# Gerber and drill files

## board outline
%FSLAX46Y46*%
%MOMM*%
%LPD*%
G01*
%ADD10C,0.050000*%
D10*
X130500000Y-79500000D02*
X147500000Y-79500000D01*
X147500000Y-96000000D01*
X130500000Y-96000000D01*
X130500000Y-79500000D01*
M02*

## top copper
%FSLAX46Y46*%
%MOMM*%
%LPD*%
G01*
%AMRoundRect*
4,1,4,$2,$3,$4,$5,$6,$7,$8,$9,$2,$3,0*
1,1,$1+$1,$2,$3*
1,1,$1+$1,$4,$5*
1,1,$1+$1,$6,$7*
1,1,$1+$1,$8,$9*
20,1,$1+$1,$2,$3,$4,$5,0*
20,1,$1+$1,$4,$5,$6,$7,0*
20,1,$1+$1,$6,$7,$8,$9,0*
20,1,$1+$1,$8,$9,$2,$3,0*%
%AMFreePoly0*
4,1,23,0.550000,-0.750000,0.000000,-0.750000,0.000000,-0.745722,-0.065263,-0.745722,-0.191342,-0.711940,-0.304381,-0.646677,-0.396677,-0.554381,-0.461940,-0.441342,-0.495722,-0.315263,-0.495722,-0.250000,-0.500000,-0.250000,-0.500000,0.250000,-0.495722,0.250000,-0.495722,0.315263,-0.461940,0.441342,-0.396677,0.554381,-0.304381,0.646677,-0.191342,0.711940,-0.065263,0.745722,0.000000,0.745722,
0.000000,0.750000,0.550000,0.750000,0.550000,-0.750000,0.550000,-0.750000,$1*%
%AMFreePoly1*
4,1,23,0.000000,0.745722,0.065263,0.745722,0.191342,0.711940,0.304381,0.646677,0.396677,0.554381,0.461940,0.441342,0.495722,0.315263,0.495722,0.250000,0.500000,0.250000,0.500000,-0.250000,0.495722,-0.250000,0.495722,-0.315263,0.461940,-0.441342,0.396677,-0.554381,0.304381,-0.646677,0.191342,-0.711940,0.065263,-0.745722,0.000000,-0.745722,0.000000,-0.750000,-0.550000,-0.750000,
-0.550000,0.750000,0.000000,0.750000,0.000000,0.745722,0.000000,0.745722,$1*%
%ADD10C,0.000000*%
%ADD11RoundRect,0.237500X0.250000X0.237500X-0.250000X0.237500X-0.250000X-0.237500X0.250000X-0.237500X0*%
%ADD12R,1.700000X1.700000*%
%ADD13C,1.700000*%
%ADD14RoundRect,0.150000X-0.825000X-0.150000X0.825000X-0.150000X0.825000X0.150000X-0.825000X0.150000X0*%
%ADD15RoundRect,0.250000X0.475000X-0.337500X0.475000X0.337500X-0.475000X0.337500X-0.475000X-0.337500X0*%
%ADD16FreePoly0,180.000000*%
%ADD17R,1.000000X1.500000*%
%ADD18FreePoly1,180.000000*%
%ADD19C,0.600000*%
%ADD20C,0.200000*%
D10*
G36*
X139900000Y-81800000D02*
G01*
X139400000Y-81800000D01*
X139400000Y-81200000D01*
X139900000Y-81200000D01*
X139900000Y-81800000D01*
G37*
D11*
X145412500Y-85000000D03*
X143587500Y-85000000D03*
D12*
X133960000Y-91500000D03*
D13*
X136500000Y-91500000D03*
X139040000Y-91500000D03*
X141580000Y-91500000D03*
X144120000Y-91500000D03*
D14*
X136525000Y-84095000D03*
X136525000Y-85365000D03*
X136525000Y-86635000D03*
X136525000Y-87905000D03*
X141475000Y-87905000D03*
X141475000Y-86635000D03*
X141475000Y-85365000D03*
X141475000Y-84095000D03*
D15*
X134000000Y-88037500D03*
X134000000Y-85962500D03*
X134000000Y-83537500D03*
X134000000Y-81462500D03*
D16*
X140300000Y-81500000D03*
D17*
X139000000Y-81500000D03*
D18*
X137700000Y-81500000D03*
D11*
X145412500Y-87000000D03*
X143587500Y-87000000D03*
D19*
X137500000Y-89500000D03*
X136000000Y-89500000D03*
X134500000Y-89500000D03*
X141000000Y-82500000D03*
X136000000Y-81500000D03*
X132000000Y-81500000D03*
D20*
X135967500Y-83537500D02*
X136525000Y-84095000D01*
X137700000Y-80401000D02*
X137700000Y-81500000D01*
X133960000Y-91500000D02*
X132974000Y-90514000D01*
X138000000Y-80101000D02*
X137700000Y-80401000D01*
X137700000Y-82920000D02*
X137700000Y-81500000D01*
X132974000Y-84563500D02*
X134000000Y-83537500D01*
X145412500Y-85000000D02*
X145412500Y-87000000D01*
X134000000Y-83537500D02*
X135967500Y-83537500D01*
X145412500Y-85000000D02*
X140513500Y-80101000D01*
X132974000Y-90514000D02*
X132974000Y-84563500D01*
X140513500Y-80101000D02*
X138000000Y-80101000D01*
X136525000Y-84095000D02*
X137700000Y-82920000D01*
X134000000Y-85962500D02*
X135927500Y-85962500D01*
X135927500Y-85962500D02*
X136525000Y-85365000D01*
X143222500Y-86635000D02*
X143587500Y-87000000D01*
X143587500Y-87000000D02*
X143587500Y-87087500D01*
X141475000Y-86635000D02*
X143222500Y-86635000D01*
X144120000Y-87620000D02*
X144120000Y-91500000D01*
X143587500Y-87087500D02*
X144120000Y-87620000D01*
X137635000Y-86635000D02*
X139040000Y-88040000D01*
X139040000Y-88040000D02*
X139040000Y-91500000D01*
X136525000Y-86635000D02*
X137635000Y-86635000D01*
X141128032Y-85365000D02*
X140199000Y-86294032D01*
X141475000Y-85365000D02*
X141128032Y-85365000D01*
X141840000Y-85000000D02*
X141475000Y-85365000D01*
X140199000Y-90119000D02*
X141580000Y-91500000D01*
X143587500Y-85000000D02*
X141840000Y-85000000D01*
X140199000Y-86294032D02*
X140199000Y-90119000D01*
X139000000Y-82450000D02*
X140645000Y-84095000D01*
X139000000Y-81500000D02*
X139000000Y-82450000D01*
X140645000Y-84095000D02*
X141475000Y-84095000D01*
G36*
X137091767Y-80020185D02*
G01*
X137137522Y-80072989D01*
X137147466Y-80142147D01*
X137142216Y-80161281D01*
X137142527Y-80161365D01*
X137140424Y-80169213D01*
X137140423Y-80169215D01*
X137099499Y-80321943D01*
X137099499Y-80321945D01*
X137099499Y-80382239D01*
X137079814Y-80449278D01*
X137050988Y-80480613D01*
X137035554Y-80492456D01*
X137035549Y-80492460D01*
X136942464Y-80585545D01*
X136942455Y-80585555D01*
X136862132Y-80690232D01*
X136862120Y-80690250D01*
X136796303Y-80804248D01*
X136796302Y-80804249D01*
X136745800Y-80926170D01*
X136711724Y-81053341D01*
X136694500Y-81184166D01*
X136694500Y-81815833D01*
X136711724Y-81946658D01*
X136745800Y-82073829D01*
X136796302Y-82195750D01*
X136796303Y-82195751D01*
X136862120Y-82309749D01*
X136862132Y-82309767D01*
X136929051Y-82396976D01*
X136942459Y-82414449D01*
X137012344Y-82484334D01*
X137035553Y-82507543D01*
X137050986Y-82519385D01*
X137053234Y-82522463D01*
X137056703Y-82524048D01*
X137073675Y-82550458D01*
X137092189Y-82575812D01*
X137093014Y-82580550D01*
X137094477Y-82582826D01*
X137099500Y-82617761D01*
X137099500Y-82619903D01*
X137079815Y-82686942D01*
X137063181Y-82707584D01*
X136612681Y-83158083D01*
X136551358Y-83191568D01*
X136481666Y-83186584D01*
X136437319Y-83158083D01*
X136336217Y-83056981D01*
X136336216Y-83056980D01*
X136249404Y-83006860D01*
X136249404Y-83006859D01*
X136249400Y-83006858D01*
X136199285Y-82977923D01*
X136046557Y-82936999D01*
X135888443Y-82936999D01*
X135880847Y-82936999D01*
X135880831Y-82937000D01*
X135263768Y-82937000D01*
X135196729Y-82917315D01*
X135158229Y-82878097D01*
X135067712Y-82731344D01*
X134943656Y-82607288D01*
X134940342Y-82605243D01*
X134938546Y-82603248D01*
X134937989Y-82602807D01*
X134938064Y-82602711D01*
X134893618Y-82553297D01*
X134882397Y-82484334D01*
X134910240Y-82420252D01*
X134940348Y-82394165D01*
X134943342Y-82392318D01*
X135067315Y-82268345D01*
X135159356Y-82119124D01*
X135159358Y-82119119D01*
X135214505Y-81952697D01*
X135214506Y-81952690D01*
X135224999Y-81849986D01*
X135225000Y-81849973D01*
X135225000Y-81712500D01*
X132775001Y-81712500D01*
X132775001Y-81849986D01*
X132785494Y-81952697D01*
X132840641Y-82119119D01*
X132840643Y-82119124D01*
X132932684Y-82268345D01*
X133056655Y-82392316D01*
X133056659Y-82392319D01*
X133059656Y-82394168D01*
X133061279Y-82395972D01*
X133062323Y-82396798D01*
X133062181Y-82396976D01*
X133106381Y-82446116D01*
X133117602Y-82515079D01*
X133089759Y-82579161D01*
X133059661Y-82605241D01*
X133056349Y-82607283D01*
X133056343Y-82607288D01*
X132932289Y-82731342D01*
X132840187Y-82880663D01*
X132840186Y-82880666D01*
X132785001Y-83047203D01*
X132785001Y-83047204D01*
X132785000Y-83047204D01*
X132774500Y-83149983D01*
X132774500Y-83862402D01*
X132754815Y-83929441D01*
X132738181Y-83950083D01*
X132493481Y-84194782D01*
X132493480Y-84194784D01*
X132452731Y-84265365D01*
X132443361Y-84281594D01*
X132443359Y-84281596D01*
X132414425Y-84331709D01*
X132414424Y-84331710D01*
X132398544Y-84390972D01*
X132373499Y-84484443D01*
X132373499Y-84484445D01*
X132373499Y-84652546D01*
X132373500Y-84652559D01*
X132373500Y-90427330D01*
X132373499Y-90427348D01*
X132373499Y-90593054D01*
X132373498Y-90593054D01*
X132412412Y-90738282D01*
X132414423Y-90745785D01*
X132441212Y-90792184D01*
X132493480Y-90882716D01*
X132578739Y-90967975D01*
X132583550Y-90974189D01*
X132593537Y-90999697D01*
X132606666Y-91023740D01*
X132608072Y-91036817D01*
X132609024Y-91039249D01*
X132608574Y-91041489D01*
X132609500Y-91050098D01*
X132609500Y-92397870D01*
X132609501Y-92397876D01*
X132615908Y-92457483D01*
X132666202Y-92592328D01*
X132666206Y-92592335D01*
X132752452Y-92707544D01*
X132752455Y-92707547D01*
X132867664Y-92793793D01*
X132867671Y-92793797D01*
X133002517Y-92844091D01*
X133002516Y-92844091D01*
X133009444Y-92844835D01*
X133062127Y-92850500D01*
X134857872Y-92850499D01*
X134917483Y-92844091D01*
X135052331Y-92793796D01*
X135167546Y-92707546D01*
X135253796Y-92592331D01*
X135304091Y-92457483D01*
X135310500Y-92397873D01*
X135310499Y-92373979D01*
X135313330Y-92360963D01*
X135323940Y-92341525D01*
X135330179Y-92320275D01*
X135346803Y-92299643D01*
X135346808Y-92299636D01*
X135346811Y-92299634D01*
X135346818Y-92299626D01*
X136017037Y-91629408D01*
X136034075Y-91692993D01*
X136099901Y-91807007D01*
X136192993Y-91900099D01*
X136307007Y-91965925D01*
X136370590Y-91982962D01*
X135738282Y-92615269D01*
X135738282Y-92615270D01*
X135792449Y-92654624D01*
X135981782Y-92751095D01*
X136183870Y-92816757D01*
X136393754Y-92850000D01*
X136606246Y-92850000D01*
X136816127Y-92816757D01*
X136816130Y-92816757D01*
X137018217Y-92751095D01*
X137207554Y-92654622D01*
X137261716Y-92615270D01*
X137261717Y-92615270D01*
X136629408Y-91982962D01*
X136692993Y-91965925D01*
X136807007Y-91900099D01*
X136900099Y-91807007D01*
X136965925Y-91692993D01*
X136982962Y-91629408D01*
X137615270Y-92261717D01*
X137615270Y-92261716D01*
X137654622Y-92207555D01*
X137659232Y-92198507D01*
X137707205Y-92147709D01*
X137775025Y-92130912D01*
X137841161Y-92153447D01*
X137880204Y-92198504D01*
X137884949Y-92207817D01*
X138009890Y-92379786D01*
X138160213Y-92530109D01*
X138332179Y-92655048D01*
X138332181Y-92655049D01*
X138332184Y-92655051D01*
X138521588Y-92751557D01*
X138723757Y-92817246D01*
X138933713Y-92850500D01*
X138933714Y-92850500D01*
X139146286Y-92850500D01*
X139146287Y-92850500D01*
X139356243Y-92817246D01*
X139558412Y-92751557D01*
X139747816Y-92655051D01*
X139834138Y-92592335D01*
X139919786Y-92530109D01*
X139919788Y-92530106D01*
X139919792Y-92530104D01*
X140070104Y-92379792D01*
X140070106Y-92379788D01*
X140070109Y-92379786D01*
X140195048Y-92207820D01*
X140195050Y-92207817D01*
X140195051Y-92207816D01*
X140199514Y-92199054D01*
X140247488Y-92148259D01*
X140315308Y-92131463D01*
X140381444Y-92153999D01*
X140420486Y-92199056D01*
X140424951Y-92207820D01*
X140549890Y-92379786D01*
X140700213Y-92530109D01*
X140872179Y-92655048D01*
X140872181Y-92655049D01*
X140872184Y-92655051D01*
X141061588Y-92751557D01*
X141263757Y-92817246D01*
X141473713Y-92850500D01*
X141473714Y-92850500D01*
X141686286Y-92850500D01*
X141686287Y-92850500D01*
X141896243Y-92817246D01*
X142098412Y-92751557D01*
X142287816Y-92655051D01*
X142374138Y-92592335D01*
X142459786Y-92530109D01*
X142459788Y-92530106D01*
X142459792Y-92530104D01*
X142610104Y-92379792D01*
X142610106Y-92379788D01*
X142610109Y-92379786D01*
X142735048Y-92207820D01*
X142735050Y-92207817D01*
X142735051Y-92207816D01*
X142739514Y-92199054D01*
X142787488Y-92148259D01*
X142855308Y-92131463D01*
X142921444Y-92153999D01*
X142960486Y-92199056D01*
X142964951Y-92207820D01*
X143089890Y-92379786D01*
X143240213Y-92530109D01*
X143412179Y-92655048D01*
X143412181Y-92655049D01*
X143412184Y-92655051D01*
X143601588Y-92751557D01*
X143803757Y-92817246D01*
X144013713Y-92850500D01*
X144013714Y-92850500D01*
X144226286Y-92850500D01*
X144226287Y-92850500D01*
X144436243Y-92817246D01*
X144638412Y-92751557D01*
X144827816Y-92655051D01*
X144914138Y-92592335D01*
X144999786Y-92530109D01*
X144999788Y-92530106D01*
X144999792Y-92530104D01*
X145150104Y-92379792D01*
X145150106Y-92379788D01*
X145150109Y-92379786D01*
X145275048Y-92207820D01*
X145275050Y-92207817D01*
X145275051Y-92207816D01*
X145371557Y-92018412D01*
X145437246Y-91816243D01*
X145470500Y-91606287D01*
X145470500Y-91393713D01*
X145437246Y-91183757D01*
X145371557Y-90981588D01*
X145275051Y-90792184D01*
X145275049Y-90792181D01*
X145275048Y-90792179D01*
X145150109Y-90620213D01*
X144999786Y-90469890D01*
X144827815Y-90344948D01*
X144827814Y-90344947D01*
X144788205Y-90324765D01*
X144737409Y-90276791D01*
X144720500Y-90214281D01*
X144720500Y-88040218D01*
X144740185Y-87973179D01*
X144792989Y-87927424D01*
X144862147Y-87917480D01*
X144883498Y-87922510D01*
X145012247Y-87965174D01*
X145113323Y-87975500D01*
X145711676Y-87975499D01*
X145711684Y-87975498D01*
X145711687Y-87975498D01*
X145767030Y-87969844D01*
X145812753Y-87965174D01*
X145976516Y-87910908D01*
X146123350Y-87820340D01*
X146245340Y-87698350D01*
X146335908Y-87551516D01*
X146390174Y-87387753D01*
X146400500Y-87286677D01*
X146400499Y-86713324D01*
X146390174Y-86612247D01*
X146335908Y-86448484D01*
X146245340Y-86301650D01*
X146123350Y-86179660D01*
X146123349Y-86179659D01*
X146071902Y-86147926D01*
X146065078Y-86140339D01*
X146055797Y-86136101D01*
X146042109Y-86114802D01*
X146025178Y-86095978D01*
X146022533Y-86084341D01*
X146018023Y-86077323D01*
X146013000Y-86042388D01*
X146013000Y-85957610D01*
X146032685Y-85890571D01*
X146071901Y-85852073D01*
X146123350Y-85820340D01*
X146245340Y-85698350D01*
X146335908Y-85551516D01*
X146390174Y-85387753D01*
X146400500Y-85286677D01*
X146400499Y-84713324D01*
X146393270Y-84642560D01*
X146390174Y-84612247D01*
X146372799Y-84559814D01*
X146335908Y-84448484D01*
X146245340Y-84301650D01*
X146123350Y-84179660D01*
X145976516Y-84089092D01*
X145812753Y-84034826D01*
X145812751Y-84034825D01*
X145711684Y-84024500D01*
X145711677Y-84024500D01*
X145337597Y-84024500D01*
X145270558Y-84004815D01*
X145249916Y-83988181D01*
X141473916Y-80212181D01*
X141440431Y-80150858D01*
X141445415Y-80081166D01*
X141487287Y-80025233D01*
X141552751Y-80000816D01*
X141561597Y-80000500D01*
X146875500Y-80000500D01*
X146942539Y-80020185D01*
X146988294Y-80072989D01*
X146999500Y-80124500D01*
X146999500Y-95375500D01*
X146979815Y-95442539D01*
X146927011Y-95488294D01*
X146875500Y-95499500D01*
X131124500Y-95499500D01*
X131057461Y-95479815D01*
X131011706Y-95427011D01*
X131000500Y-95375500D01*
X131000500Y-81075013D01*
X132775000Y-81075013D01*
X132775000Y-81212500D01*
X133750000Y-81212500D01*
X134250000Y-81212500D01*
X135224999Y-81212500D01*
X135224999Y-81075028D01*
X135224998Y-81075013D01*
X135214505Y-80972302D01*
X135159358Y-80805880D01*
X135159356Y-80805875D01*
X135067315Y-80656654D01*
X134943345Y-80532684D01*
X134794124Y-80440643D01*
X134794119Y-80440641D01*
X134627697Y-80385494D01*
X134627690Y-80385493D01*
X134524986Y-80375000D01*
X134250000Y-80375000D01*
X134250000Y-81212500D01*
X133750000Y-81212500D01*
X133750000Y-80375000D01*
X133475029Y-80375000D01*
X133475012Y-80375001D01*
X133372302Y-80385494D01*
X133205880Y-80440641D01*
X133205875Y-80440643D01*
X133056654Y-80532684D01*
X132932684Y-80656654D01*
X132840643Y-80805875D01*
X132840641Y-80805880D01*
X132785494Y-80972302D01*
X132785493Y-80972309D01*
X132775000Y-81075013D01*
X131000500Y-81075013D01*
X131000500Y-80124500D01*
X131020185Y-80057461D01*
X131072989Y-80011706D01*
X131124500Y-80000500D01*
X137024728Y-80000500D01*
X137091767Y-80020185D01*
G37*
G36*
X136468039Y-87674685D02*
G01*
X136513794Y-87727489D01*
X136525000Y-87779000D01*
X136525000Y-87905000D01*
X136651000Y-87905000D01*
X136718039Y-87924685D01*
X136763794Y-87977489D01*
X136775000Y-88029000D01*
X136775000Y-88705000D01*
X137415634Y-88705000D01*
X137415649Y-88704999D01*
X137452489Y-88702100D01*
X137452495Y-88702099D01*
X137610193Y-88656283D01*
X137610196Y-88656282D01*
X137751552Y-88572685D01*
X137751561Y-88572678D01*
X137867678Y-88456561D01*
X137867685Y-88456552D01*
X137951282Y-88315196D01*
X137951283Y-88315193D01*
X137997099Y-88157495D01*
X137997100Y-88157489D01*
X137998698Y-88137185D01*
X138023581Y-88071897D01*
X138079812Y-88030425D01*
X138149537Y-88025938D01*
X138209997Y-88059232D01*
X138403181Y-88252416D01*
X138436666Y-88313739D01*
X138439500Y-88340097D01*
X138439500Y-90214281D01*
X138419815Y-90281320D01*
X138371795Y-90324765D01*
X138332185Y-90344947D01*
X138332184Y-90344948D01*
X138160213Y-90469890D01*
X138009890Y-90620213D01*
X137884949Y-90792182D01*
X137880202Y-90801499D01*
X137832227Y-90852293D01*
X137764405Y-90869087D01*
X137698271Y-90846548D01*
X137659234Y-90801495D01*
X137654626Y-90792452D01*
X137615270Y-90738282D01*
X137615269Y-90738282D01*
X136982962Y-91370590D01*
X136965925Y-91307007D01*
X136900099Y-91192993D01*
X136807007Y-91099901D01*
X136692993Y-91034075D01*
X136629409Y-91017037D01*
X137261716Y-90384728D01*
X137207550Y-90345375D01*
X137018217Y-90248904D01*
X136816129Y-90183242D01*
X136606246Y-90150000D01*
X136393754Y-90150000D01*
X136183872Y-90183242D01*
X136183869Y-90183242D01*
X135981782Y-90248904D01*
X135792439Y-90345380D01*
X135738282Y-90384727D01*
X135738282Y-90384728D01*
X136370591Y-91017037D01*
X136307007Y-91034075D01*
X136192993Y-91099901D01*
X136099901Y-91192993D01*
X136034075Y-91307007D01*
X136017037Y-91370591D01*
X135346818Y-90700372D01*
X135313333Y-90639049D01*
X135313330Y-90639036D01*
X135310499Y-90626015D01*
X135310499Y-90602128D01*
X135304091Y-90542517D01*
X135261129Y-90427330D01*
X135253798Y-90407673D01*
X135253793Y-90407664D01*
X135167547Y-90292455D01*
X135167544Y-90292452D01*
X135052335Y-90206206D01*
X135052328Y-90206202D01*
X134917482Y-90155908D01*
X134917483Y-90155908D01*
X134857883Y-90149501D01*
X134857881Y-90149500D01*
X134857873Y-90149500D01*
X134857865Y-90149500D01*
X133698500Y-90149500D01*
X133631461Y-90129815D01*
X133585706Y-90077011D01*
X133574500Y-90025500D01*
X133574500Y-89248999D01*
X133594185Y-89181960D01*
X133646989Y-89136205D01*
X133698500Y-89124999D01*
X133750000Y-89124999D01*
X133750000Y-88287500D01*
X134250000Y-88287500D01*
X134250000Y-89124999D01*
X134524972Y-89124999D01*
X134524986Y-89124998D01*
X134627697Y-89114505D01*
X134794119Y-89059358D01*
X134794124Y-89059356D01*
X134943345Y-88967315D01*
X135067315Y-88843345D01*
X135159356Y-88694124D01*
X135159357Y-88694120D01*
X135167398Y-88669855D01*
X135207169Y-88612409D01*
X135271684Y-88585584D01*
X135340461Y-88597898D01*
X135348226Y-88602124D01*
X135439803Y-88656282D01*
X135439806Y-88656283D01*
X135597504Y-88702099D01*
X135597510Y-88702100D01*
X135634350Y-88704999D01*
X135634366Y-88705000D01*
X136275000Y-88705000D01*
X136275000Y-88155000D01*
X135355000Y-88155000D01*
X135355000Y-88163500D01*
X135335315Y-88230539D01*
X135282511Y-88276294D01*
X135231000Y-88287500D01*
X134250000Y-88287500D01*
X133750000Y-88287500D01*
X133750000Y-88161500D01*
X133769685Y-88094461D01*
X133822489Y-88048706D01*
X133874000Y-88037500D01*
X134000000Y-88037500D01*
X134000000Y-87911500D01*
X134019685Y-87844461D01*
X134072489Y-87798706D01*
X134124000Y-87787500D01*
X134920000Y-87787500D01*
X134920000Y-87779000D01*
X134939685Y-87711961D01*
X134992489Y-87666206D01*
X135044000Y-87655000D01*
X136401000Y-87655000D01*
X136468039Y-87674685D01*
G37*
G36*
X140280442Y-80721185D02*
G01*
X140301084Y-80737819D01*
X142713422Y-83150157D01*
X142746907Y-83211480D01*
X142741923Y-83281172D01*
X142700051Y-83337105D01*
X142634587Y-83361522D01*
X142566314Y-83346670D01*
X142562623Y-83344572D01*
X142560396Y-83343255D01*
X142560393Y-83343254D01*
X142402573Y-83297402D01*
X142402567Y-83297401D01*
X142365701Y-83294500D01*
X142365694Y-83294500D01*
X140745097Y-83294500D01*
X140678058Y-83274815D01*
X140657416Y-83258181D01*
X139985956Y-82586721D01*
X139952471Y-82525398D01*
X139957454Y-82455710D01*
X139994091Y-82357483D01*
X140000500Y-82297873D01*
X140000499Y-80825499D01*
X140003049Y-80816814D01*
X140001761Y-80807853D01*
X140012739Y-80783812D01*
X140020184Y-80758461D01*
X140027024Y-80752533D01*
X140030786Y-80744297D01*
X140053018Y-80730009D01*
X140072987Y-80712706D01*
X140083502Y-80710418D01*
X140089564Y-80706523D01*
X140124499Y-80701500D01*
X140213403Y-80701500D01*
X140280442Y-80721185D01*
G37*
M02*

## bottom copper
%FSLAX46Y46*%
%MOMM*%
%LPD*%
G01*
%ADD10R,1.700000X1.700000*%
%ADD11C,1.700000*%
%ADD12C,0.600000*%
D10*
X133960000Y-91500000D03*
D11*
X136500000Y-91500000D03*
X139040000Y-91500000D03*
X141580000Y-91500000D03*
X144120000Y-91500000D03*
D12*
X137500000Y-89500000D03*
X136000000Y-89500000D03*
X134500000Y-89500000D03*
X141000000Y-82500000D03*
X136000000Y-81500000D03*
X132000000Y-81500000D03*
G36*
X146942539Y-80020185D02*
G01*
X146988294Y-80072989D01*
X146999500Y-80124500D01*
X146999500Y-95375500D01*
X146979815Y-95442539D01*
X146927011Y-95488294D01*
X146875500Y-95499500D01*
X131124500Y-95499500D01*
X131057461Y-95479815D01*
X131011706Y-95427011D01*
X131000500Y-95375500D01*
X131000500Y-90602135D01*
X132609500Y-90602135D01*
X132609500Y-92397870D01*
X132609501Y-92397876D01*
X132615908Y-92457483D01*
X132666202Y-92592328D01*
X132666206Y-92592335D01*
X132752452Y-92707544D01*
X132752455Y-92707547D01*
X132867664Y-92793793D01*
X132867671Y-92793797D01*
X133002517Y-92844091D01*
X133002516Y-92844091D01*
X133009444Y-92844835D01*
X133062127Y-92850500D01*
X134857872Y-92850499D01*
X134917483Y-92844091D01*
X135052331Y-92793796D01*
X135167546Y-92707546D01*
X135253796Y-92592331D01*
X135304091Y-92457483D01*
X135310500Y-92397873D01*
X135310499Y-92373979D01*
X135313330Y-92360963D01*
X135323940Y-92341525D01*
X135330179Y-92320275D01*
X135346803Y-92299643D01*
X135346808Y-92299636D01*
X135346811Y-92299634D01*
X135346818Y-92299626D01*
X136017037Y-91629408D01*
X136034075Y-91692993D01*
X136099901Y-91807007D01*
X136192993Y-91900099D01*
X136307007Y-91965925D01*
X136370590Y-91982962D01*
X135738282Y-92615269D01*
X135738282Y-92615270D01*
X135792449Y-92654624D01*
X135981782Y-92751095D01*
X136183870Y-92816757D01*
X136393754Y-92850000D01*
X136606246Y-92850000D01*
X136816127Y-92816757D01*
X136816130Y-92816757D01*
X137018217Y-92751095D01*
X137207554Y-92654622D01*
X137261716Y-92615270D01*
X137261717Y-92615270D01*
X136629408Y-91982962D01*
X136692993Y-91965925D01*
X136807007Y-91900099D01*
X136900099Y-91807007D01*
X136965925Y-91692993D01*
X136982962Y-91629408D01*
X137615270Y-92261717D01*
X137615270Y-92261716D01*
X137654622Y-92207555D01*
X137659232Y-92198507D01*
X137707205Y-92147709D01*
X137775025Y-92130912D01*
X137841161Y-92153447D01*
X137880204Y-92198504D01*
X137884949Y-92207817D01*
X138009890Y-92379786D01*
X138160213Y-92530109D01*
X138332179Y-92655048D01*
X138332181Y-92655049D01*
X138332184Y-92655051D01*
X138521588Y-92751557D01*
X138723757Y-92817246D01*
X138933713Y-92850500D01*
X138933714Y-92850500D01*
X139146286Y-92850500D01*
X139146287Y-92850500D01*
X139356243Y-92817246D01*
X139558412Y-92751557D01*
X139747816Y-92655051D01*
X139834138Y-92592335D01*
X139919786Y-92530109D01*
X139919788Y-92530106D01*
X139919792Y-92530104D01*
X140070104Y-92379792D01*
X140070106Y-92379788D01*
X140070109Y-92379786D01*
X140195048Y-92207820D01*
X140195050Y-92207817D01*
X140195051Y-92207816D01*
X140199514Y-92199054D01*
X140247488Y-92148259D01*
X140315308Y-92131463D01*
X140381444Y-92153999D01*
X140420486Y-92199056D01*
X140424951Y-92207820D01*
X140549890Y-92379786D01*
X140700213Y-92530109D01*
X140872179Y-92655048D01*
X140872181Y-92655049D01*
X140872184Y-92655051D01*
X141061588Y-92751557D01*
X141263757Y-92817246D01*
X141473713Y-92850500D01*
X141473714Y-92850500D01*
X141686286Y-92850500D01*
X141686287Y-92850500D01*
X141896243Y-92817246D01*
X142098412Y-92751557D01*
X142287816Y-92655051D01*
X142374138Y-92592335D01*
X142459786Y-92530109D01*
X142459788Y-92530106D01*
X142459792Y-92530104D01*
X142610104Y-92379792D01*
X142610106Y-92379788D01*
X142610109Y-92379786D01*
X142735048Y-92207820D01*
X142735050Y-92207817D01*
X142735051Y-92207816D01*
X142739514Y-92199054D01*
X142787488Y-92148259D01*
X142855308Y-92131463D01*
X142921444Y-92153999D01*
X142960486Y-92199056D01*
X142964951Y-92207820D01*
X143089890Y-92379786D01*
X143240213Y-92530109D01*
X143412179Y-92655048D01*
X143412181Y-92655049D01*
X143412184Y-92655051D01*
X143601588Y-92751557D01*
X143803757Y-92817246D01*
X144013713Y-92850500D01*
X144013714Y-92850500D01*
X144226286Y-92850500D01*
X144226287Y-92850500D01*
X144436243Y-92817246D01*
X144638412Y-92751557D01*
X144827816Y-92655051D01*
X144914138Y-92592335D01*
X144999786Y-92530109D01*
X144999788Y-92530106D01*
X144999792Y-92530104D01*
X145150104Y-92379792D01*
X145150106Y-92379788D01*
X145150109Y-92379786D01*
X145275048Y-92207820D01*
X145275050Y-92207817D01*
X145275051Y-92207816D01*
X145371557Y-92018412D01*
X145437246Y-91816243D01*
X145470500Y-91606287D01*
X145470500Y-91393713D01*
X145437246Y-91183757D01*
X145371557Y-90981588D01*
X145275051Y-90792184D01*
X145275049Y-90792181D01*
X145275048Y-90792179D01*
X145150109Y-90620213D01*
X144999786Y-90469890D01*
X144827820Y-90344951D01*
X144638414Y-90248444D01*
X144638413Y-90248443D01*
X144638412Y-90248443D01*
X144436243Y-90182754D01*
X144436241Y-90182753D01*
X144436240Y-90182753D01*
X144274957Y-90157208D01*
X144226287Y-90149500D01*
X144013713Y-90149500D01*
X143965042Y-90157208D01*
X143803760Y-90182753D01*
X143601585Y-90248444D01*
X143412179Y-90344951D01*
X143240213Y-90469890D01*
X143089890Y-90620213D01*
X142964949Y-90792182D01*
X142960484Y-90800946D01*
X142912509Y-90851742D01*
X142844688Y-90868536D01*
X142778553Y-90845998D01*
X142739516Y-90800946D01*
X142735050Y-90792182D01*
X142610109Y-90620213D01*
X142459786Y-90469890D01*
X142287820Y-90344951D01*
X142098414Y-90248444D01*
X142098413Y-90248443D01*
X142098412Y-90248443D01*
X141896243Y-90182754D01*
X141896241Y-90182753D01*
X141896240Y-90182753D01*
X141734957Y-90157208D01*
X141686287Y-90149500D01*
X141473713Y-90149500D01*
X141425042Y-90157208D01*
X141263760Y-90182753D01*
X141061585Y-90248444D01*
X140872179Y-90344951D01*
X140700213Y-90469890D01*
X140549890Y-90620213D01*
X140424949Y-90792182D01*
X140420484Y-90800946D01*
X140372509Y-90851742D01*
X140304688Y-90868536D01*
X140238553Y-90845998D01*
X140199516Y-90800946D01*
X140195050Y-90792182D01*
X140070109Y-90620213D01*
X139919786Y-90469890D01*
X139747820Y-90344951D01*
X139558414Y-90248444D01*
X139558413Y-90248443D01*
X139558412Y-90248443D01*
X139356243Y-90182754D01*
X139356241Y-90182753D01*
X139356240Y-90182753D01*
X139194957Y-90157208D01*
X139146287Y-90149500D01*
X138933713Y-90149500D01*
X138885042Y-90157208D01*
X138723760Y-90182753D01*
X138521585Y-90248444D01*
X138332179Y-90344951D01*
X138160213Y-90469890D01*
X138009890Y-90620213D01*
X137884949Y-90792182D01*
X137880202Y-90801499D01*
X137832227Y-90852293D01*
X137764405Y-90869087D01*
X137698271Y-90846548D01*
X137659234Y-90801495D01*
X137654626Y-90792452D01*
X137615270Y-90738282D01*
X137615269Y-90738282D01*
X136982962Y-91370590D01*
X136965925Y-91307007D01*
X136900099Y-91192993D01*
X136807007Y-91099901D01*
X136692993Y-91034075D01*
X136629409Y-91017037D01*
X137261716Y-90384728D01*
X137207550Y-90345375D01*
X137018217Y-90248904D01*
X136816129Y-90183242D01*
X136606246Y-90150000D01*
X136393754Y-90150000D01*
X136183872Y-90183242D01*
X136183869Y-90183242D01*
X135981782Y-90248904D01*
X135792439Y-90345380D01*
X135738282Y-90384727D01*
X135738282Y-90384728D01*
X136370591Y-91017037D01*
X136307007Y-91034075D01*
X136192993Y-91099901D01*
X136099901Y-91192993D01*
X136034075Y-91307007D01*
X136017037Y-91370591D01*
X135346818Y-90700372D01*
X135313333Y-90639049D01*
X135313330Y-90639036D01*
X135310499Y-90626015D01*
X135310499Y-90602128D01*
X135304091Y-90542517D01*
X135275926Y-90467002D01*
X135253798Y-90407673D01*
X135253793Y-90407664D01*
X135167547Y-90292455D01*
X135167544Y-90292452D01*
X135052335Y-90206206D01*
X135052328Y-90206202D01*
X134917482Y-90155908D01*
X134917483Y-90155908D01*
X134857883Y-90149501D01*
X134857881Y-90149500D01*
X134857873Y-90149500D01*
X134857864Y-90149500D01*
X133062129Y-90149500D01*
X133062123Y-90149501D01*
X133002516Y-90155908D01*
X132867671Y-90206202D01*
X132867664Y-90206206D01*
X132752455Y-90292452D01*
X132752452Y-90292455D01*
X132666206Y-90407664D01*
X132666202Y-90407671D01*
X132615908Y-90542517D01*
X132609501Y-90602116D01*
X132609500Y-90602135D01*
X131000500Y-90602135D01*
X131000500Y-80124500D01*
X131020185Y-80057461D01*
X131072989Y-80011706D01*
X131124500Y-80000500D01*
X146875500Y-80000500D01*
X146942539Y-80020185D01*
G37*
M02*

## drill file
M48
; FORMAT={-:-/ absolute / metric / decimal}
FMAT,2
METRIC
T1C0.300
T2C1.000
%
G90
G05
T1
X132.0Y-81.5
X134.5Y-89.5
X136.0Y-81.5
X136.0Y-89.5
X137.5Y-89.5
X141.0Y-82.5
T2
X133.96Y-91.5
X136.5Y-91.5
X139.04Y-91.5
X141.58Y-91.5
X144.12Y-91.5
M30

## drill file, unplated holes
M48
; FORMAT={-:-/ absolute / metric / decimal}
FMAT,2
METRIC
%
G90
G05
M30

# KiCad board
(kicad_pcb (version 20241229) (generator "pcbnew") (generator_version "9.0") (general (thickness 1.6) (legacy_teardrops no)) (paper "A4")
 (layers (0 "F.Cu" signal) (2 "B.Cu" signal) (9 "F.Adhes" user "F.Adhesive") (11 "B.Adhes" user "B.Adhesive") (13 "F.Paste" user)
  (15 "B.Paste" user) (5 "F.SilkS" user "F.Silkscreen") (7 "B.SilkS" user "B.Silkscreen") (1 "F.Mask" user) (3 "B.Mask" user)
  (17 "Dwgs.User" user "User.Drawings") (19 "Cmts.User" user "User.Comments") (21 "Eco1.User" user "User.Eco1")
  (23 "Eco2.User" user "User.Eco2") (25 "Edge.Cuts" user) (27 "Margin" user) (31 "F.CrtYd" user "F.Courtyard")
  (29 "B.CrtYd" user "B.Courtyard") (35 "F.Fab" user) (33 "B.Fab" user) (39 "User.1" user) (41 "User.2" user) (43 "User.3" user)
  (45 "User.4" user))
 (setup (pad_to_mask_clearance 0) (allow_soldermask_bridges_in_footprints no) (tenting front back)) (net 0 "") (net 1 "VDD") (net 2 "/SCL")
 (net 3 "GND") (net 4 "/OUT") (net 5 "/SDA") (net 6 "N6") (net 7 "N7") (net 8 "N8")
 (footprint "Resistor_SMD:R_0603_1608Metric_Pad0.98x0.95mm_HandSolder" (layer "F.Cu") (at 144.5 85 180)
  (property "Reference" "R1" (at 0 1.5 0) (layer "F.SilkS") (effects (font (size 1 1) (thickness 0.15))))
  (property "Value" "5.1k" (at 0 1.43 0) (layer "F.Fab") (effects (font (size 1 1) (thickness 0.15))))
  (pad "1" smd roundrect (at -0.9125 0 180) (size 0.975 0.95) (layers "F.Cu" "F.Mask" "F.Paste") (roundrect_rratio 0.25) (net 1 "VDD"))
  (pad "2" smd roundrect (at 0.9125 0 180) (size 0.975 0.95) (layers "F.Cu" "F.Mask" "F.Paste") (roundrect_rratio 0.25) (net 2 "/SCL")))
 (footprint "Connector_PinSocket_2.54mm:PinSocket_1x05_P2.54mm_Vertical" (layer "F.Cu") (at 133.96 91.5 90)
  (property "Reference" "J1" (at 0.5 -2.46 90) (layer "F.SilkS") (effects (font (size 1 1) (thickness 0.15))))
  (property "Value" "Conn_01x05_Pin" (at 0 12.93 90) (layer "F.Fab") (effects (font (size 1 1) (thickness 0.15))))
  (pad "1" thru_hole rect (at 0 0 90) (size 1.7 1.7) (drill 1) (layers "*.Cu" "*.Mask") (remove_unused_layers no) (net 1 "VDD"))
  (pad "2" thru_hole circle (at 0 2.54 90) (size 1.7 1.7) (drill 1) (layers "*.Cu" "*.Mask") (remove_unused_layers no) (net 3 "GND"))
  (pad "3" thru_hole circle (at 0 5.08 90) (size 1.7 1.7) (drill 1) (layers "*.Cu" "*.Mask") (remove_unused_layers no) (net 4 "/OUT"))
  (pad "4" thru_hole circle (at 0 7.62 90) (size 1.7 1.7) (drill 1) (layers "*.Cu" "*.Mask") (remove_unused_layers no) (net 2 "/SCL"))
  (pad "5" thru_hole circle (at 0 10.16 90) (size 1.7 1.7) (drill 1) (layers "*.Cu" "*.Mask") (remove_unused_layers no) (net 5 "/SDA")))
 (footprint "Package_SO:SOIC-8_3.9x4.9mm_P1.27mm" (layer "F.Cu") (at 139 86)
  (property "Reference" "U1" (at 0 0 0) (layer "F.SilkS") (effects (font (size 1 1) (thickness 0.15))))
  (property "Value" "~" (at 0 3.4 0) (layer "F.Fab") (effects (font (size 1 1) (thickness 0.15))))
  (pad "1" smd roundrect (at -2.475 -1.905) (size 1.95 0.6) (layers "F.Cu" "F.Mask" "F.Paste") (roundrect_rratio 0.25) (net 1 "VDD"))
  (pad "2" smd roundrect (at -2.475 -0.635) (size 1.95 0.6) (layers "F.Cu" "F.Mask" "F.Paste") (roundrect_rratio 0.25) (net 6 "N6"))
  (pad "3" smd roundrect (at -2.475 0.635) (size 1.95 0.6) (layers "F.Cu" "F.Mask" "F.Paste") (roundrect_rratio 0.25) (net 4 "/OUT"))
  (pad "4" smd roundrect (at -2.475 1.905) (size 1.95 0.6) (layers "F.Cu" "F.Mask" "F.Paste") (roundrect_rratio 0.25) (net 3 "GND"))
  (pad "5" smd roundrect (at 2.475 1.905) (size 1.95 0.6) (layers "F.Cu" "F.Mask" "F.Paste") (roundrect_rratio 0.25) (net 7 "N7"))
  (pad "6" smd roundrect (at 2.475 0.635) (size 1.95 0.6) (layers "F.Cu" "F.Mask" "F.Paste") (roundrect_rratio 0.25) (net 5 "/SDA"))
  (pad "7" smd roundrect (at 2.475 -0.635) (size 1.95 0.6) (layers "F.Cu" "F.Mask" "F.Paste") (roundrect_rratio 0.25) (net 2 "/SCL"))
  (pad "8" smd roundrect (at 2.475 -1.905) (size 1.95 0.6) (layers "F.Cu" "F.Mask" "F.Paste") (roundrect_rratio 0.25) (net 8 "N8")))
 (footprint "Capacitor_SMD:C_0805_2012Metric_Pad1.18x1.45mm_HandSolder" (layer "F.Cu") (at 134 87 90)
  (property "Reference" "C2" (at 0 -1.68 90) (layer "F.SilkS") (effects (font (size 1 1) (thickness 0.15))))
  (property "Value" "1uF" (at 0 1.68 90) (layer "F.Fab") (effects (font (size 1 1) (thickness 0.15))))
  (pad "1" smd roundrect (at -1.0375 0 90) (size 1.175 1.45) (layers "F.Cu" "F.Mask" "F.Paste") (roundrect_rratio 0.212766) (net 3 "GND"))
  (pad "2" smd roundrect (at 1.0375 0 90) (size 1.175 1.45) (layers "F.Cu" "F.Mask" "F.Paste") (roundrect_rratio 0.212766) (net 6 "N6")))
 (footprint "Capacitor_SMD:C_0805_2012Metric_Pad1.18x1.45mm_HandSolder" (layer "F.Cu") (at 134 82.5 90)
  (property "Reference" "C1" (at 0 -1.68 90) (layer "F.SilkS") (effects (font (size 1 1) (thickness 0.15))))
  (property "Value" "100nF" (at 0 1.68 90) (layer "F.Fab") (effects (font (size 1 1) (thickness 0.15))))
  (pad "1" smd roundrect (at -1.0375 0 90) (size 1.175 1.45) (layers "F.Cu" "F.Mask" "F.Paste") (roundrect_rratio 0.212766) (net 1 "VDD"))
  (pad "2" smd roundrect (at 1.0375 0 90) (size 1.175 1.45) (layers "F.Cu" "F.Mask" "F.Paste") (roundrect_rratio 0.212766) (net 3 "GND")))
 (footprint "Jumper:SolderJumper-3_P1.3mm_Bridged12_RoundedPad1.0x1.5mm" (layer "F.Cu") (at 139 81.5 180)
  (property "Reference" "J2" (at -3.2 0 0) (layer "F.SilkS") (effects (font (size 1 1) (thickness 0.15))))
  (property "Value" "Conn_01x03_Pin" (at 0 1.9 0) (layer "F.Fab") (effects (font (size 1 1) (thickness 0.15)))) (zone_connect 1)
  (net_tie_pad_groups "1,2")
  (fp_poly (pts (xy -0.9 -0.3) (xy -0.4 -0.3) (xy -0.4 0.3) (xy -0.9 0.3)) (stroke (width 0) (type solid)) (fill yes) (layer "F.Cu"))
  (pad "1" smd custom (at -1.3 0 180) (size 1 0.5) (layers "F.Cu" "F.Mask") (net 3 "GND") (zone_connect 2) (thermal_bridge_angle 45)
   (options (clearance outline) (anchor rect)) (primitives))
  (pad "2" smd rect (at 0 0 180) (size 1 1.5) (layers "F.Cu" "F.Mask") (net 8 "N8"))
  (pad "3" smd custom (at 1.3 0 180) (size 1 0.5) (layers "F.Cu" "F.Mask") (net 1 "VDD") (zone_connect 2) (thermal_bridge_angle 45)
   (options (clearance outline) (anchor rect)) (primitives)))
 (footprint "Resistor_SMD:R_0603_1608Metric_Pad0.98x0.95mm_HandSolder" (layer "F.Cu") (at 144.5 87 180)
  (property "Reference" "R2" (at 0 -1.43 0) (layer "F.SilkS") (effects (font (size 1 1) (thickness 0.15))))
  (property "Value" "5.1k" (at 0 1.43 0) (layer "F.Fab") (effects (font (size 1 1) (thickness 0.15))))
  (pad "1" smd roundrect (at -0.9125 0 180) (size 0.975 0.95) (layers "F.Cu" "F.Mask" "F.Paste") (roundrect_rratio 0.25) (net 1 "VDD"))
  (pad "2" smd roundrect (at 0.9125 0 180) (size 0.975 0.95) (layers "F.Cu" "F.Mask" "F.Paste") (roundrect_rratio 0.25) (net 5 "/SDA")))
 (gr_rect (start 130.5 79.5) (end 147.5 96) (stroke (width 0.05) (type default)) (fill no) (layer "Edge.Cuts"))
 (segment (start 135.9675 83.5375) (end 136.525 84.095) (width 0.2) (layer "F.Cu") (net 1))
 (segment (start 137.7 80.401) (end 137.7 81.5) (width 0.2) (layer "F.Cu") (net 1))
 (segment (start 133.96 91.5) (end 132.974 90.514) (width 0.2) (layer "F.Cu") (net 1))
 (segment (start 138 80.101) (end 137.7 80.401) (width 0.2) (layer "F.Cu") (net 1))
 (segment (start 137.7 82.92) (end 137.7 81.5) (width 0.2) (layer "F.Cu") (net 1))
 (segment (start 132.974 84.5635) (end 134 83.5375) (width 0.2) (layer "F.Cu") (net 1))
 (segment (start 145.4125 85) (end 145.4125 87) (width 0.2) (layer "F.Cu") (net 1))
 (segment (start 134 83.5375) (end 135.9675 83.5375) (width 0.2) (layer "F.Cu") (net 1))
 (segment (start 145.4125 85) (end 140.5135 80.101) (width 0.2) (layer "F.Cu") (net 1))
 (segment (start 132.974 90.514) (end 132.974 84.5635) (width 0.2) (layer "F.Cu") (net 1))
 (segment (start 140.5135 80.101) (end 138 80.101) (width 0.2) (layer "F.Cu") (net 1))
 (segment (start 136.525 84.095) (end 137.7 82.92) (width 0.2) (layer "F.Cu") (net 1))
 (via (at 137.5 89.5) (size 0.6) (drill 0.3) (layers "F.Cu" "B.Cu") (free yes) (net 3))
 (via (at 136 89.5) (size 0.6) (drill 0.3) (layers "F.Cu" "B.Cu") (free yes) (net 3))
 (via (at 134.5 89.5) (size 0.6) (drill 0.3) (layers "F.Cu" "B.Cu") (free yes) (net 3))
 (via (at 141 82.5) (size 0.6) (drill 0.3) (layers "F.Cu" "B.Cu") (free yes) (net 3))
 (via (at 136 81.5) (size 0.6) (drill 0.3) (layers "F.Cu" "B.Cu") (free yes) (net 3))
 (via (at 132 81.5) (size 0.6) (drill 0.3) (layers "F.Cu" "B.Cu") (free yes) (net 3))
 (segment (start 134 85.9625) (end 135.9275 85.9625) (width 0.2) (layer "F.Cu") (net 6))
 (segment (start 135.9275 85.9625) (end 136.525 85.365) (width 0.2) (layer "F.Cu") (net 6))
 (segment (start 143.2225 86.635) (end 143.5875 87) (width 0.2) (layer "F.Cu") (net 5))
 (segment (start 143.5875 87) (end 143.5875 87.0875) (width 0.2) (layer "F.Cu") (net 5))
 (segment (start 141.475 86.635) (end 143.2225 86.635) (width 0.2) (layer "F.Cu") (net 5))
 (segment (start 144.12 87.62) (end 144.12 91.5) (width 0.2) (layer "F.Cu") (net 5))
 (segment (start 143.5875 87.0875) (end 144.12 87.62) (width 0.2) (layer "F.Cu") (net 5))
 (segment (start 137.635 86.635) (end 139.04 88.04) (width 0.2) (layer "F.Cu") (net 4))
 (segment (start 139.04 88.04) (end 139.04 91.5) (width 0.2) (layer "F.Cu") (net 4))
 (segment (start 136.525 86.635) (end 137.635 86.635) (width 0.2) (layer "F.Cu") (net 4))
 (segment (start 141.128032 85.365) (end 140.199 86.294032) (width 0.2) (layer "F.Cu") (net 2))
 (segment (start 141.475 85.365) (end 141.128032 85.365) (width 0.2) (layer "F.Cu") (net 2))
 (segment (start 141.84 85) (end 141.475 85.365) (width 0.2) (layer "F.Cu") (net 2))
 (segment (start 140.199 90.119) (end 141.58 91.5) (width 0.2) (layer "F.Cu") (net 2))
 (segment (start 143.5875 85) (end 141.84 85) (width 0.2) (layer "F.Cu") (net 2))
 (segment (start 140.199 86.294032) (end 140.199 90.119) (width 0.2) (layer "F.Cu") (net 2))
 (segment (start 139 82.45) (end 140.645 84.095) (width 0.2) (layer "F.Cu") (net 8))
 (segment (start 139 81.5) (end 139 82.45) (width 0.2) (layer "F.Cu") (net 8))
 (segment (start 140.645 84.095) (end 141.475 84.095) (width 0.2) (layer "F.Cu") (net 8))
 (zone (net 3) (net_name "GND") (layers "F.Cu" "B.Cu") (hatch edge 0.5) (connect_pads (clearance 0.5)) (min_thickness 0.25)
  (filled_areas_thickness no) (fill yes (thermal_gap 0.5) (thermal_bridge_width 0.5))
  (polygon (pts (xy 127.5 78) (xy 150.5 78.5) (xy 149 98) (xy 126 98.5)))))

